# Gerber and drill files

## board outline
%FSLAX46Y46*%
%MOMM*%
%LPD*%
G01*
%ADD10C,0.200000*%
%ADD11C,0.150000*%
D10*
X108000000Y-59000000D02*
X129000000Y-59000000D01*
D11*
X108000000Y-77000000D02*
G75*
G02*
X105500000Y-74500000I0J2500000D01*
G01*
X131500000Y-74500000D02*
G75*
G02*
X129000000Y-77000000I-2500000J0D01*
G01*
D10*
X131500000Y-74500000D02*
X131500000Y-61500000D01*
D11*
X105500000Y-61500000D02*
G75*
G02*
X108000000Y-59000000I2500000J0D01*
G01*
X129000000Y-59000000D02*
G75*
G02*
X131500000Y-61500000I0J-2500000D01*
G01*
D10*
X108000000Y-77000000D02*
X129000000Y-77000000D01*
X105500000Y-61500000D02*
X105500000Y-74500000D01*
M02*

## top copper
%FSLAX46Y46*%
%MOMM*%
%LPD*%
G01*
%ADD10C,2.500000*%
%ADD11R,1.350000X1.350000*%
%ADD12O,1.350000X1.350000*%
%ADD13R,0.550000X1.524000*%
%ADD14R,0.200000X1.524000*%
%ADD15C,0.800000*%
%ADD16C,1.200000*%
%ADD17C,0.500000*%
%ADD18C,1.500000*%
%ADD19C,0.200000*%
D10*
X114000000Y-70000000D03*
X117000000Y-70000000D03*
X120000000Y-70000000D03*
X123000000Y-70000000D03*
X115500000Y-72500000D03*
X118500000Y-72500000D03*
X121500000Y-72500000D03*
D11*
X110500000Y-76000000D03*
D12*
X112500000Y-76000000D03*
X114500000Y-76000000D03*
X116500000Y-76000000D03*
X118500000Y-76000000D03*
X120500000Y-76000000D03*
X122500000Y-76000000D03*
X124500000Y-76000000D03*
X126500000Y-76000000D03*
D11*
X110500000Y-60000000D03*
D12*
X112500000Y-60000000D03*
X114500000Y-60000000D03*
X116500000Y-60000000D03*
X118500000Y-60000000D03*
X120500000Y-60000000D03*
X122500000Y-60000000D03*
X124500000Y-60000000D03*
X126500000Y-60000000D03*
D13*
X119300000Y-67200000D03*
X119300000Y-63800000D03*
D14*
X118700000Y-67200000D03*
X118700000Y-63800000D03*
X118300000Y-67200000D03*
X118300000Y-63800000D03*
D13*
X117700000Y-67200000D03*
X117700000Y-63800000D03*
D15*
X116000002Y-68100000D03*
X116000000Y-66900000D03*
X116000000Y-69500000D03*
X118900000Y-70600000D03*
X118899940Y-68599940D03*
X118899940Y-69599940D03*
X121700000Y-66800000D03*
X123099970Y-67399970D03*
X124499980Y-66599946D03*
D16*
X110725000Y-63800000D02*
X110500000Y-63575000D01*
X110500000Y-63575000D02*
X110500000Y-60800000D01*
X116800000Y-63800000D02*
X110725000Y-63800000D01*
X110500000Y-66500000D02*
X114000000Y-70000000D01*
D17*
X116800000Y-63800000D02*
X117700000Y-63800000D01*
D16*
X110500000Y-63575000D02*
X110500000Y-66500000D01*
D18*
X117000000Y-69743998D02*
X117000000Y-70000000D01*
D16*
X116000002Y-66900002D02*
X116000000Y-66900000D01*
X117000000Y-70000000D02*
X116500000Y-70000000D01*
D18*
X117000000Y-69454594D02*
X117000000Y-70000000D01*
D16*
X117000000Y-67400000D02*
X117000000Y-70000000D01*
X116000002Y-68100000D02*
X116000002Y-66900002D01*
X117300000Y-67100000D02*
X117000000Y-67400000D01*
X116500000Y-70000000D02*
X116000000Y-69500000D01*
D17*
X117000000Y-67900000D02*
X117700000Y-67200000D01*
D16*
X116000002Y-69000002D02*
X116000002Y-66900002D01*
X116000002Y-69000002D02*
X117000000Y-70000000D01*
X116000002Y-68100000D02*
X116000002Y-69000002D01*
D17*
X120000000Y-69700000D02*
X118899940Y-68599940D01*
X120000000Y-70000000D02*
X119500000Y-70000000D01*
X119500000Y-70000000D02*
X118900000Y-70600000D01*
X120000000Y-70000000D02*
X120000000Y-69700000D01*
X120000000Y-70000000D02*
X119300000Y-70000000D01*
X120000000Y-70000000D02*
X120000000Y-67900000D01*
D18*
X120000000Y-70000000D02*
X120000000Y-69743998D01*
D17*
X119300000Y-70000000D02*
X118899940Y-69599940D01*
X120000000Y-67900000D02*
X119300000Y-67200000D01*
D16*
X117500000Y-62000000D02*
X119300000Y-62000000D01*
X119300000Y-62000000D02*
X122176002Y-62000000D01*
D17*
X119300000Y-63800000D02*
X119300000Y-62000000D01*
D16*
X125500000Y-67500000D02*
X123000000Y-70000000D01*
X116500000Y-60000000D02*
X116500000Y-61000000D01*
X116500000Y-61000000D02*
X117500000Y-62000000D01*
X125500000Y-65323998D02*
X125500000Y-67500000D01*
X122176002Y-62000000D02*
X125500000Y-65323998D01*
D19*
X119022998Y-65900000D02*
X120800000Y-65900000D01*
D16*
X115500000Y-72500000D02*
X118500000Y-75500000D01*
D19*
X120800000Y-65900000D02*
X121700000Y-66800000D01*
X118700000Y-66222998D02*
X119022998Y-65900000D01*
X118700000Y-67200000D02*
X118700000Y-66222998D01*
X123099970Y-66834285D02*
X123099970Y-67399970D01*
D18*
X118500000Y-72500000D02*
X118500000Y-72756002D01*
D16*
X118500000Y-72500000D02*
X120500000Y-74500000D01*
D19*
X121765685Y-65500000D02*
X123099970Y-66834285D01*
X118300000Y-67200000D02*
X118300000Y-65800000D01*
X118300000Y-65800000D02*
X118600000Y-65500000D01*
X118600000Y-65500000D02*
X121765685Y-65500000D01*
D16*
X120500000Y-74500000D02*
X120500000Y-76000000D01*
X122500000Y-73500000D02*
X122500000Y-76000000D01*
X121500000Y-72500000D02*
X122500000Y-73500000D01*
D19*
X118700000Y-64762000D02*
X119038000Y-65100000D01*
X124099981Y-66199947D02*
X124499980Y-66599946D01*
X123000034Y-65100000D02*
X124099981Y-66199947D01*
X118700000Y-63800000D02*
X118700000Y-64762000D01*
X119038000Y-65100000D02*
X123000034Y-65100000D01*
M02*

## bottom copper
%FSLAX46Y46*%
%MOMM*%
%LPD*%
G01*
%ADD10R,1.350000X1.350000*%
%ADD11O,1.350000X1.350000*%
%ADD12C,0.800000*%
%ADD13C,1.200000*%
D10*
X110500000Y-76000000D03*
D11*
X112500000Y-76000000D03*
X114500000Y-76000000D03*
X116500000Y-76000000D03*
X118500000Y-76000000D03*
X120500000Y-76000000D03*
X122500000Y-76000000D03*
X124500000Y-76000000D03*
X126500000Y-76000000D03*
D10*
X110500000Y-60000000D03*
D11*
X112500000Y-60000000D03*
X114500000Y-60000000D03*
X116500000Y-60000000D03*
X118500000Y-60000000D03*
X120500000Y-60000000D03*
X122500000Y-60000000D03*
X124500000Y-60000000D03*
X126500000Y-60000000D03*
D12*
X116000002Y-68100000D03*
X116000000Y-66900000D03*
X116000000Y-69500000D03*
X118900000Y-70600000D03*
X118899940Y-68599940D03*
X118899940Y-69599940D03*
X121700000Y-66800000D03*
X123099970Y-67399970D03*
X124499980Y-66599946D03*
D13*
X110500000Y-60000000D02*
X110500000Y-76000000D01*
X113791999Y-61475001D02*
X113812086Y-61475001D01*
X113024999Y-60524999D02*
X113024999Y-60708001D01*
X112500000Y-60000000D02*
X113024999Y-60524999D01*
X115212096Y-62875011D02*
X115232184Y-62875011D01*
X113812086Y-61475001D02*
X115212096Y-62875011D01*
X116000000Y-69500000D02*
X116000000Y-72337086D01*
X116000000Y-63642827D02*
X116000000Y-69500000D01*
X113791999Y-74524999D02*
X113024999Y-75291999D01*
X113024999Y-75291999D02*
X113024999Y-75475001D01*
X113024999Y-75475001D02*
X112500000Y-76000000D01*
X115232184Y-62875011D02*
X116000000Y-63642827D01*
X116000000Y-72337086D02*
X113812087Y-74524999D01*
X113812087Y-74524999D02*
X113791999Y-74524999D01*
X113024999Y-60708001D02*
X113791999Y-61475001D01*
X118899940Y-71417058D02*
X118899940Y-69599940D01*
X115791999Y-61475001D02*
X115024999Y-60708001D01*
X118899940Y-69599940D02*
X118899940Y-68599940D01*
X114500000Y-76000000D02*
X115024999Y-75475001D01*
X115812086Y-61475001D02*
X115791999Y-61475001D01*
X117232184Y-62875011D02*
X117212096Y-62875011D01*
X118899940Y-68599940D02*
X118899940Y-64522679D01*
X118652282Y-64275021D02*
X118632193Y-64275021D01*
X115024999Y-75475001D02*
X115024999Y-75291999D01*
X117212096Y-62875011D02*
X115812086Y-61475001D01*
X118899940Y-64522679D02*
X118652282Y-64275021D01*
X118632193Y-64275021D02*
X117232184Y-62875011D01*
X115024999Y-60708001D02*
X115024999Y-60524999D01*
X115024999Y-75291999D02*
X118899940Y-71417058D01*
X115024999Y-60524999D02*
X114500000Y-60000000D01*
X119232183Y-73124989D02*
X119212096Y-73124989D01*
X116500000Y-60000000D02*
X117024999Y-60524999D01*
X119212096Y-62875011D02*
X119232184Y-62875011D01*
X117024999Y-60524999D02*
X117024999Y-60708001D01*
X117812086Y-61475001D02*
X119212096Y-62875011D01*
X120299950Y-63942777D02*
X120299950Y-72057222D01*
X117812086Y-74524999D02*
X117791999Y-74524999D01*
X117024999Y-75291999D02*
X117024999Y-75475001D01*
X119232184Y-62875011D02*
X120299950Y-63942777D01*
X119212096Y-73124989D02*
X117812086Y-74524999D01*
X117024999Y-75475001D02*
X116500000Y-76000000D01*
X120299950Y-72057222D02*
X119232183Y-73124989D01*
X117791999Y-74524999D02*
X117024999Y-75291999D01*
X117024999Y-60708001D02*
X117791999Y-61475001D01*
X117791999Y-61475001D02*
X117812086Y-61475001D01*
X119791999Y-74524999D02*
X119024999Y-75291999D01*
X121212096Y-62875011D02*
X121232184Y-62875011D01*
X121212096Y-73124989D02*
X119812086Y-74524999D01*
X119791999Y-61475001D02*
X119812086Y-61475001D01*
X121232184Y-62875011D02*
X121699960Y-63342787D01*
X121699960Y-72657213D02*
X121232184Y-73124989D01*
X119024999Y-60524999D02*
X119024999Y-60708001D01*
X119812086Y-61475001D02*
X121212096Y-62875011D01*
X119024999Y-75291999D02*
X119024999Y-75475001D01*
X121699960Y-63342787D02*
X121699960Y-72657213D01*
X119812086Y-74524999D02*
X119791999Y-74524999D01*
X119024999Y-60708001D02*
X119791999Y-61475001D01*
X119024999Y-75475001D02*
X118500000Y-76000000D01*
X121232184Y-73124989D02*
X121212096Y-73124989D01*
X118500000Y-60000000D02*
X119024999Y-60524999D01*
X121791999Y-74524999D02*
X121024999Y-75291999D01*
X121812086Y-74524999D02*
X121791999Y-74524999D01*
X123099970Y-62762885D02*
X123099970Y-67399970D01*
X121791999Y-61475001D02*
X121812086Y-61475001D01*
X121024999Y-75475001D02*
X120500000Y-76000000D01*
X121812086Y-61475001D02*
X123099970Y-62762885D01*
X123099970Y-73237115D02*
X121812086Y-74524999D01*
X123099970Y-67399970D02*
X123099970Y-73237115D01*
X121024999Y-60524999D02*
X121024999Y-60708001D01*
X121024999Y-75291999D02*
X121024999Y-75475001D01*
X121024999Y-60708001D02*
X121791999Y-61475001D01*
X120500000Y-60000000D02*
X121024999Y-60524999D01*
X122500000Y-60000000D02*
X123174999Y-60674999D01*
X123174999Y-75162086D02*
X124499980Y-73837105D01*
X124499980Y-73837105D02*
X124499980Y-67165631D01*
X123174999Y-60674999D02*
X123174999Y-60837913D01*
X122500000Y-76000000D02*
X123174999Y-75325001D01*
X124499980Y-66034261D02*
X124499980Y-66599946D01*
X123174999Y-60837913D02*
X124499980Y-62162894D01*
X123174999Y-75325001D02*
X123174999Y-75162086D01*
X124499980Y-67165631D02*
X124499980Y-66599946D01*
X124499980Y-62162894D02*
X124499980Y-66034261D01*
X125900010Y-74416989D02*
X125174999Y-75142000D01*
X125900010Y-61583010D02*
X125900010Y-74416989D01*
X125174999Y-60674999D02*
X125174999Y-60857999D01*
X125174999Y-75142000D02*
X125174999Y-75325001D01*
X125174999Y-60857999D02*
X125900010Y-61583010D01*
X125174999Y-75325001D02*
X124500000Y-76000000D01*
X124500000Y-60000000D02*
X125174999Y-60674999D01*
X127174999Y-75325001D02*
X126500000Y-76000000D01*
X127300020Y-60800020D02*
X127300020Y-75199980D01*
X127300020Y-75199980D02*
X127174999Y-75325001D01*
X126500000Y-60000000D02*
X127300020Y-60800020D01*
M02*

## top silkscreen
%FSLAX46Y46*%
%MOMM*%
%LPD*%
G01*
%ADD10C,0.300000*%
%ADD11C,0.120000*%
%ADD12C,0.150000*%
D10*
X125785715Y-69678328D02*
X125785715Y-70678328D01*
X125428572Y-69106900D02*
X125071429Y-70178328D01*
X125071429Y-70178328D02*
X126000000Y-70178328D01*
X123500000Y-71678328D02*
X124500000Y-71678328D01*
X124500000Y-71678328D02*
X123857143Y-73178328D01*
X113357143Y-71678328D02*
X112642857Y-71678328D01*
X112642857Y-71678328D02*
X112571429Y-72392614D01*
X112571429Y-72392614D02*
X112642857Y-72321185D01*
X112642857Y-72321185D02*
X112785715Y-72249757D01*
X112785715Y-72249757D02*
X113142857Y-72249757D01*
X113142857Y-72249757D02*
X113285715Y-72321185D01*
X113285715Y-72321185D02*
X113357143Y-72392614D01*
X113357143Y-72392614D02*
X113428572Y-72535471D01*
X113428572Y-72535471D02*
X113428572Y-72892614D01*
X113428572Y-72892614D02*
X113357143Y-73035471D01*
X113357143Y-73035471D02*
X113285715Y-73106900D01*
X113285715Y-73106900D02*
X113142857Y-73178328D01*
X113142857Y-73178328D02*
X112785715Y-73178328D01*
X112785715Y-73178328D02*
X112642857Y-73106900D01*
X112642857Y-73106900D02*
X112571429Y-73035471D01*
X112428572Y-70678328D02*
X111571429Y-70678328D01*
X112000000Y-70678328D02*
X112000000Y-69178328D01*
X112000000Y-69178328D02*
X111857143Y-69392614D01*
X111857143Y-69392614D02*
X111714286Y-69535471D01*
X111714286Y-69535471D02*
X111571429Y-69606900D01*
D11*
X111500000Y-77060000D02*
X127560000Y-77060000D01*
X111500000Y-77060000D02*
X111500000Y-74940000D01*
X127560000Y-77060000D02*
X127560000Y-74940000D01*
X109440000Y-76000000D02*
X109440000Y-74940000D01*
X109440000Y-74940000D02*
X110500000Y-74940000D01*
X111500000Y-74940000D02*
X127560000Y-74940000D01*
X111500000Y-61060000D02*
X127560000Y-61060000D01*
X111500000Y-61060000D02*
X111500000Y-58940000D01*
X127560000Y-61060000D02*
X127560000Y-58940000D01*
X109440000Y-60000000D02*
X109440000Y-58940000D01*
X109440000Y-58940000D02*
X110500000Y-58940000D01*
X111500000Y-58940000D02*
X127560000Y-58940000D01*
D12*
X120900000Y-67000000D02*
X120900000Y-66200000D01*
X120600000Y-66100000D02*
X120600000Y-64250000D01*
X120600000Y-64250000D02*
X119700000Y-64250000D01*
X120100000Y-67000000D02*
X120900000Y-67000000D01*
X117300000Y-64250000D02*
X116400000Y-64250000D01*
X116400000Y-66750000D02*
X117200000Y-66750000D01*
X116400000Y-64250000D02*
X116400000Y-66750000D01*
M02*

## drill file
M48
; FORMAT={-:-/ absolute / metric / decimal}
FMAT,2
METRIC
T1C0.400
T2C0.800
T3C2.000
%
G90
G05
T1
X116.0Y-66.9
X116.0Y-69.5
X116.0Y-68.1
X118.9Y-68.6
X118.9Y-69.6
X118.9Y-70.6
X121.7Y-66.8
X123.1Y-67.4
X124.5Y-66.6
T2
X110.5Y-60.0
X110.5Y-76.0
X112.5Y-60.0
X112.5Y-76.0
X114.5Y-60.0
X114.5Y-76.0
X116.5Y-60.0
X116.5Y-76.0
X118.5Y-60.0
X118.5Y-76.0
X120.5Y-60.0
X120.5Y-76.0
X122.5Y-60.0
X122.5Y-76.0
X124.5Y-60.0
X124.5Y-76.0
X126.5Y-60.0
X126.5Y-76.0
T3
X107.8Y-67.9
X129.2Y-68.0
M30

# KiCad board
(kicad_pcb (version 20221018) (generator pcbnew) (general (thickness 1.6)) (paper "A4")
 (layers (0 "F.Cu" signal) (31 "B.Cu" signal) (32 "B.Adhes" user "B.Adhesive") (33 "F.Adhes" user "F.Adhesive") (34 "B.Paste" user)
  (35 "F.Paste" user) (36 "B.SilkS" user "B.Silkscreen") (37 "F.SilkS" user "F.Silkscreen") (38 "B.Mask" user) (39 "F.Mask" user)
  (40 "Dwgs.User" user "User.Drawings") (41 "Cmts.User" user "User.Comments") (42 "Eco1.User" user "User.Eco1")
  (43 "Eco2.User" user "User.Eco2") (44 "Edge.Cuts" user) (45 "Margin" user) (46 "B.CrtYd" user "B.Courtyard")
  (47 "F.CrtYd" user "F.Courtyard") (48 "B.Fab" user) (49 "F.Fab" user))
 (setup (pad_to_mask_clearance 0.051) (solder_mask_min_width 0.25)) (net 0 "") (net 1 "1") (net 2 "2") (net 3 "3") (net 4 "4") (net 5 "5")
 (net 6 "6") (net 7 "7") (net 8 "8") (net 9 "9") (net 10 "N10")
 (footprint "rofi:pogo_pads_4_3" (layer "F.Cu") (at 118.5 70)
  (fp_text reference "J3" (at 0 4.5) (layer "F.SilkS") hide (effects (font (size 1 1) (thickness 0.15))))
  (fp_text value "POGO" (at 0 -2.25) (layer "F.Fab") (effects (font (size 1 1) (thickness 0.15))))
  (pad "1" smd circle (at -4.5 0) (size 2.5 2.5) (layers "F.Cu" "F.Paste" "F.Mask") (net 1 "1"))
  (pad "2" smd circle (at -1.5 0) (size 2.5 2.5) (layers "F.Cu" "F.Paste" "F.Mask") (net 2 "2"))
  (pad "3" smd circle (at 1.5 0) (size 2.5 2.5) (layers "F.Cu" "F.Paste" "F.Mask") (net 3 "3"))
  (pad "4" smd circle (at 4.5 0) (size 2.5 2.5) (layers "F.Cu" "F.Paste" "F.Mask") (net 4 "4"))
  (pad "5" smd circle (at -3 2.5) (size 2.5 2.5) (layers "F.Cu" "F.Paste" "F.Mask") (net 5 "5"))
  (pad "6" smd circle (at 0 2.5) (size 2.5 2.5) (layers "F.Cu" "F.Paste" "F.Mask") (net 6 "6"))
  (pad "7" smd circle (at 3 2.5) (size 2.5 2.5) (layers "F.Cu" "F.Paste" "F.Mask") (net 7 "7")))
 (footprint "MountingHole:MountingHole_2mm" (layer "F.Cu") (at 129.2 68)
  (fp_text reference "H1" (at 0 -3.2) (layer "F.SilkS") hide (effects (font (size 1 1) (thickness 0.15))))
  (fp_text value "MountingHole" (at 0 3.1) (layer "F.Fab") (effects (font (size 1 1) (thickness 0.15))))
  (pad "" np_thru_hole circle (at 0 0) (size 2 2) (drill 2) (layers "*.Cu" "*.Mask")))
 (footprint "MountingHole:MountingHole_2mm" (layer "F.Cu") (at 107.8 67.9)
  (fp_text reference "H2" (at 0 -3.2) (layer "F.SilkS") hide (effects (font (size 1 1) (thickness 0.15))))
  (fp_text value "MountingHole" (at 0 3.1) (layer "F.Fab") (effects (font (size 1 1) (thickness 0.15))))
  (pad "" np_thru_hole circle (at 0 0) (size 2 2) (drill 2) (layers "*.Cu" "*.Mask")))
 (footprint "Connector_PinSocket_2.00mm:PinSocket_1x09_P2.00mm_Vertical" (layer "F.Cu") (at 110.5 76 90)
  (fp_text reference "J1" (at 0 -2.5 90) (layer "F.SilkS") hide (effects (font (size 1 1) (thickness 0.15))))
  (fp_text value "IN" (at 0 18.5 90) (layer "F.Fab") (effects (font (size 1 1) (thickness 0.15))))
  (fp_line (start -1.06 1) (end -1.06 17.06) (stroke (width 0.12) (type solid)) (layer "F.SilkS"))
  (fp_line (start -1.06 1) (end 1.06 1) (stroke (width 0.12) (type solid)) (layer "F.SilkS"))
  (fp_line (start -1.06 17.06) (end 1.06 17.06) (stroke (width 0.12) (type solid)) (layer "F.SilkS"))
  (fp_line (start 0 -1.06) (end 1.06 -1.06) (stroke (width 0.12) (type solid)) (layer "F.SilkS"))
  (fp_line (start 1.06 -1.06) (end 1.06 0) (stroke (width 0.12) (type solid)) (layer "F.SilkS"))
  (fp_line (start 1.06 1) (end 1.06 17.06) (stroke (width 0.12) (type solid)) (layer "F.SilkS"))
  (pad "1" thru_hole rect (at 0 0 90) (size 1.35 1.35) (drill 0.8) (layers "*.Cu" "*.Mask") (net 1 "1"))
  (pad "2" thru_hole oval (at 0 2 90) (size 1.35 1.35) (drill 0.8) (layers "*.Cu" "*.Mask") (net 2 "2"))
  (pad "3" thru_hole oval (at 0 4 90) (size 1.35 1.35) (drill 0.8) (layers "*.Cu" "*.Mask") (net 3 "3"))
  (pad "4" thru_hole oval (at 0 6 90) (size 1.35 1.35) (drill 0.8) (layers "*.Cu" "*.Mask") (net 4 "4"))
  (pad "5" thru_hole oval (at 0 8 90) (size 1.35 1.35) (drill 0.8) (layers "*.Cu" "*.Mask") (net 5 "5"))
  (pad "6" thru_hole oval (at 0 10 90) (size 1.35 1.35) (drill 0.8) (layers "*.Cu" "*.Mask") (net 6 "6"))
  (pad "7" thru_hole oval (at 0 12 90) (size 1.35 1.35) (drill 0.8) (layers "*.Cu" "*.Mask") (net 7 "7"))
  (pad "8" thru_hole oval (at 0 14 90) (size 1.35 1.35) (drill 0.8) (layers "*.Cu" "*.Mask") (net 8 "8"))
  (pad "9" thru_hole oval (at 0 16 90) (size 1.35 1.35) (drill 0.8) (layers "*.Cu" "*.Mask") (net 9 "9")))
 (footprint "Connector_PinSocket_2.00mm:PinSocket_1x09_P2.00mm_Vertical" (layer "F.Cu") (at 110.5 60 90)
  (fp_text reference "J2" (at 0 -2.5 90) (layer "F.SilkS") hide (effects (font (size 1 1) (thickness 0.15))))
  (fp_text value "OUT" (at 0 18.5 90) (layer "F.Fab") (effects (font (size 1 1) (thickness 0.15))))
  (fp_line (start -1.06 1) (end -1.06 17.06) (stroke (width 0.12) (type solid)) (layer "F.SilkS"))
  (fp_line (start -1.06 1) (end 1.06 1) (stroke (width 0.12) (type solid)) (layer "F.SilkS"))
  (fp_line (start -1.06 17.06) (end 1.06 17.06) (stroke (width 0.12) (type solid)) (layer "F.SilkS"))
  (fp_line (start 0 -1.06) (end 1.06 -1.06) (stroke (width 0.12) (type solid)) (layer "F.SilkS"))
  (fp_line (start 1.06 -1.06) (end 1.06 0) (stroke (width 0.12) (type solid)) (layer "F.SilkS"))
  (fp_line (start 1.06 1) (end 1.06 17.06) (stroke (width 0.12) (type solid)) (layer "F.SilkS"))
  (pad "1" thru_hole rect (at 0 0 90) (size 1.35 1.35) (drill 0.8) (layers "*.Cu" "*.Mask") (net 1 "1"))
  (pad "2" thru_hole oval (at 0 2 90) (size 1.35 1.35) (drill 0.8) (layers "*.Cu" "*.Mask") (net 2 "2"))
  (pad "3" thru_hole oval (at 0 4 90) (size 1.35 1.35) (drill 0.8) (layers "*.Cu" "*.Mask") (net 3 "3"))
  (pad "4" thru_hole oval (at 0 6 90) (size 1.35 1.35) (drill 0.8) (layers "*.Cu" "*.Mask") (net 4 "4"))
  (pad "5" thru_hole oval (at 0 8 90) (size 1.35 1.35) (drill 0.8) (layers "*.Cu" "*.Mask") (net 5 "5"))
  (pad "6" thru_hole oval (at 0 10 90) (size 1.35 1.35) (drill 0.8) (layers "*.Cu" "*.Mask") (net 6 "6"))
  (pad "7" thru_hole oval (at 0 12 90) (size 1.35 1.35) (drill 0.8) (layers "*.Cu" "*.Mask") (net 7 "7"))
  (pad "8" thru_hole oval (at 0 14 90) (size 1.35 1.35) (drill 0.8) (layers "*.Cu" "*.Mask") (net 8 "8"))
  (pad "9" thru_hole oval (at 0 16 90) (size 1.35 1.35) (drill 0.8) (layers "*.Cu" "*.Mask") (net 9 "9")))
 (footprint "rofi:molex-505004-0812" (layer "F.Cu") (at 118.5 65.5 180)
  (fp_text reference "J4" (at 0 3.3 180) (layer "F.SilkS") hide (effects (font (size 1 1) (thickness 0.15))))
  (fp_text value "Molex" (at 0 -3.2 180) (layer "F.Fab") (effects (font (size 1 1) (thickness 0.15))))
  (fp_line (start -2.4 -1.5) (end -2.4 -0.7) (stroke (width 0.15) (type solid)) (layer "F.SilkS"))
  (fp_line (start -2.1 -0.6) (end -2.1 1.25) (stroke (width 0.15) (type solid)) (layer "F.SilkS"))
  (fp_line (start -2.1 1.25) (end -1.2 1.25) (stroke (width 0.15) (type solid)) (layer "F.SilkS"))
  (fp_line (start -1.6 -1.5) (end -2.4 -1.5) (stroke (width 0.15) (type solid)) (layer "F.SilkS"))
  (fp_line (start 1.2 1.25) (end 2.1 1.25) (stroke (width 0.15) (type solid)) (layer "F.SilkS"))
  (fp_line (start 2.1 -1.25) (end 1.3 -1.25) (stroke (width 0.15) (type solid)) (layer "F.SilkS"))
  (fp_line (start 2.1 1.25) (end 2.1 -1.25) (stroke (width 0.15) (type solid)) (layer "F.SilkS"))
  (pad "1" smd rect (at -0.8 -1.7 180) (size 0.55 1.524) (layers "F.Cu" "F.Paste" "F.Mask") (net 3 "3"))
  (pad "2" smd rect (at -0.8 1.7 180) (size 0.55 1.524) (layers "F.Cu" "F.Paste" "F.Mask") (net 4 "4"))
  (pad "3" smd rect (at -0.2 -1.7 180) (size 0.2 1.524) (layers "F.Cu" "F.Paste" "F.Mask") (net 5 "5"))
  (pad "4" smd rect (at -0.2 1.7 180) (size 0.2 1.524) (layers "F.Cu" "F.Paste" "F.Mask") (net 7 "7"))
  (pad "5" smd rect (at 0.2 -1.7 180) (size 0.2 1.524) (layers "F.Cu" "F.Paste" "F.Mask") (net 6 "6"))
  (pad "6" smd rect (at 0.2 1.7 180) (size 0.2 1.524) (layers "F.Cu" "F.Paste" "F.Mask") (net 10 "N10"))
  (pad "7" smd rect (at 0.8 -1.7 180) (size 0.55 1.524) (layers "F.Cu" "F.Paste" "F.Mask") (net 2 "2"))
  (pad "8" smd rect (at 0.8 1.7 180) (size 0.55 1.524) (layers "F.Cu" "F.Paste" "F.Mask") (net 1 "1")))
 (gr_line (start 108 59) (end 129 59) (stroke (width 0.2) (type solid)) (layer "Edge.Cuts"))
 (gr_arc (start 108 77) (mid 106.232233 76.267767) (end 105.5 74.5) (stroke (width 0.15) (type solid)) (layer "Edge.Cuts"))
 (gr_arc (start 131.5 74.5) (mid 130.767767 76.267767) (end 129 77) (stroke (width 0.15) (type solid)) (layer "Edge.Cuts"))
 (gr_line (start 131.5 74.5) (end 131.5 61.5) (stroke (width 0.2) (type solid)) (layer "Edge.Cuts"))
 (gr_arc (start 105.5 61.5) (mid 106.232233 59.732233) (end 108 59) (stroke (width 0.15) (type solid)) (layer "Edge.Cuts"))
 (gr_arc (start 129 59) (mid 130.767767 59.732233) (end 131.5 61.5) (stroke (width 0.15) (type solid)) (layer "Edge.Cuts"))
 (gr_line (start 108 77) (end 129 77) (stroke (width 0.2) (type solid)) (layer "Edge.Cuts"))
 (gr_line (start 105.5 61.5) (end 105.5 74.5) (stroke (width 0.2) (type solid)) (layer "Edge.Cuts"))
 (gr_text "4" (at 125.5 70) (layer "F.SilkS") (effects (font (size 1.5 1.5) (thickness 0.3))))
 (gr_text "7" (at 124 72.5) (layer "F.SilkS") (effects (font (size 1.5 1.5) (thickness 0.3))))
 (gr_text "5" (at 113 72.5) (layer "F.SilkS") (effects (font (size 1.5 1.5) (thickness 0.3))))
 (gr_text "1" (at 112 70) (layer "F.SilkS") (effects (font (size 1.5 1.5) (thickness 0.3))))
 (segment (start 110.725 63.8) (end 110.5 63.575) (width 1.2) (layer "F.Cu") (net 1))
 (segment (start 110.5 63.575) (end 110.5 60.8) (width 1.2) (layer "F.Cu") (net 1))
 (segment (start 116.8 63.8) (end 110.725 63.8) (width 1.2) (layer "F.Cu") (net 1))
 (segment (start 110.5 66.5) (end 114 70) (width 1.2) (layer "F.Cu") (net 1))
 (segment (start 116.8 63.8) (end 117.7 63.8) (width 0.5) (layer "F.Cu") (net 1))
 (segment (start 110.5 63.575) (end 110.5 66.5) (width 1.2) (layer "F.Cu") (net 1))
 (segment (start 110.5 60) (end 110.5 76) (width 1.2) (layer "B.Cu") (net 1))
 (segment (start 117 69.743998) (end 117 70) (width 1.5) (layer "F.Cu") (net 2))
 (segment (start 116.000002 66.900002) (end 116 66.9) (width 1.2) (layer "F.Cu") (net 2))
 (segment (start 117 70) (end 116.5 70) (width 1.2) (layer "F.Cu") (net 2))
 (segment (start 117 69.454594) (end 117 70) (width 1.5) (layer "F.Cu") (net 2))
 (segment (start 117 67.4) (end 117 70) (width 1.2) (layer "F.Cu") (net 2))
 (segment (start 116.000002 68.1) (end 116.000002 66.900002) (width 1.2) (layer "F.Cu") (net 2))
 (segment (start 117.3 67.1) (end 117 67.4) (width 1.2) (layer "F.Cu") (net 2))
 (segment (start 116.5 70) (end 116 69.5) (width 1.2) (layer "F.Cu") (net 2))
 (segment (start 117 67.9) (end 117.7 67.2) (width 0.5) (layer "F.Cu") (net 2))
 (segment (start 116.000002 69.000002) (end 116.000002 66.900002) (width 1.2) (layer "F.Cu") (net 2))
 (segment (start 116.000002 69.000002) (end 117 70) (width 1.2) (layer "F.Cu") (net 2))
 (segment (start 116.000002 68.1) (end 116.000002 69.000002) (width 1.2) (layer "F.Cu") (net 2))
 (via (at 116.000002 68.1) (size 0.8) (drill 0.4) (layers "F.Cu" "B.Cu") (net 2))
 (via (at 116 66.9) (size 0.8) (drill 0.4) (layers "F.Cu" "B.Cu") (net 2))
 (via (at 116 69.5) (size 0.8) (drill 0.4) (layers "F.Cu" "B.Cu") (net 2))
 (segment (start 113.791999 61.475001) (end 113.812086 61.475001) (width 1.2) (layer "B.Cu") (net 2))
 (segment (start 113.024999 60.524999) (end 113.024999 60.708001) (width 1.2) (layer "B.Cu") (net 2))
 (segment (start 112.5 60) (end 113.024999 60.524999) (width 1.2) (layer "B.Cu") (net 2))
 (segment (start 115.212096 62.875011) (end 115.232184 62.875011) (width 1.2) (layer "B.Cu") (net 2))
 (segment (start 113.812086 61.475001) (end 115.212096 62.875011) (width 1.2) (layer "B.Cu") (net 2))
 (segment (start 116 69.5) (end 116 72.337086) (width 1.2) (layer "B.Cu") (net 2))
 (segment (start 116 63.642827) (end 116 69.5) (width 1.2) (layer "B.Cu") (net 2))
 (segment (start 113.791999 74.524999) (end 113.024999 75.291999) (width 1.2) (layer "B.Cu") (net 2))
 (segment (start 113.024999 75.291999) (end 113.024999 75.475001) (width 1.2) (layer "B.Cu") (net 2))
 (segment (start 113.024999 75.475001) (end 112.5 76) (width 1.2) (layer "B.Cu") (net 2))
 (segment (start 115.232184 62.875011) (end 116 63.642827) (width 1.2) (layer "B.Cu") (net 2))
 (segment (start 116 72.337086) (end 113.812087 74.524999) (width 1.2) (layer "B.Cu") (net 2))
 (segment (start 113.812087 74.524999) (end 113.791999 74.524999) (width 1.2) (layer "B.Cu") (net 2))
 (segment (start 113.024999 60.708001) (end 113.791999 61.475001) (width 1.2) (layer "B.Cu") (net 2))
 (segment (start 120 69.7) (end 118.89994 68.59994) (width 0.5) (layer "F.Cu") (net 3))
 (segment (start 120 70) (end 119.5 70) (width 0.5) (layer "F.Cu") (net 3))
 (segment (start 119.5 70) (end 118.9 70.6) (width 0.5) (layer "F.Cu") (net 3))
 (segment (start 120 70) (end 120 69.7) (width 0.5) (layer "F.Cu") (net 3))
 (segment (start 120 70) (end 119.3 70) (width 0.5) (layer "F.Cu") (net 3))
 (segment (start 120 70) (end 120 67.9) (width 0.5) (layer "F.Cu") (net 3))
 (segment (start 120 70) (end 120 69.743998) (width 1.5) (layer "F.Cu") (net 3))
 (segment (start 119.3 70) (end 118.89994 69.59994) (width 0.5) (layer "F.Cu") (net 3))
 (segment (start 120 67.9) (end 119.3 67.2) (width 0.5) (layer "F.Cu") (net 3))
 (via (at 118.9 70.6) (size 0.8) (drill 0.4) (layers "F.Cu" "B.Cu") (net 3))
 (via (at 118.89994 68.59994) (size 0.8) (drill 0.4) (layers "F.Cu" "B.Cu") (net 3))
 (via (at 118.89994 69.59994) (size 0.8) (drill 0.4) (layers "F.Cu" "B.Cu") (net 3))
 (segment (start 118.89994 71.417058) (end 118.89994 69.59994) (width 1.2) (layer "B.Cu") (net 3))
 (segment (start 115.791999 61.475001) (end 115.024999 60.708001) (width 1.2) (layer "B.Cu") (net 3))
 (segment (start 118.89994 69.59994) (end 118.89994 68.59994) (width 1.2) (layer "B.Cu") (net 3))
 (segment (start 114.5 76) (end 115.024999 75.475001) (width 1.2) (layer "B.Cu") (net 3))
 (segment (start 115.812086 61.475001) (end 115.791999 61.475001) (width 1.2) (layer "B.Cu") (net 3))
 (segment (start 117.232184 62.875011) (end 117.212096 62.875011) (width 1.2) (layer "B.Cu") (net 3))
 (segment (start 118.89994 68.59994) (end 118.89994 64.522679) (width 1.2) (layer "B.Cu") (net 3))
 (segment (start 118.652282 64.275021) (end 118.632193 64.275021) (width 1.2) (layer "B.Cu") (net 3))
 (segment (start 115.024999 75.475001) (end 115.024999 75.291999) (width 1.2) (layer "B.Cu") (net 3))
 (segment (start 117.212096 62.875011) (end 115.812086 61.475001) (width 1.2) (layer "B.Cu") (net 3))
 (segment (start 118.89994 64.522679) (end 118.652282 64.275021) (width 1.2) (layer "B.Cu") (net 3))
 (segment (start 118.632193 64.275021) (end 117.232184 62.875011) (width 1.2) (layer "B.Cu") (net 3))
 (segment (start 115.024999 60.708001) (end 115.024999 60.524999) (width 1.2) (layer "B.Cu") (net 3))
 (segment (start 115.024999 75.291999) (end 118.89994 71.417058) (width 1.2) (layer "B.Cu") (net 3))
 (segment (start 115.024999 60.524999) (end 114.5 60) (width 1.2) (layer "B.Cu") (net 3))
 (segment (start 117.5 62) (end 119.3 62) (width 1.2) (layer "F.Cu") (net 4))
 (segment (start 119.3 62) (end 122.176002 62) (width 1.2) (layer "F.Cu") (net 4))
 (segment (start 119.3 63.8) (end 119.3 62) (width 0.5) (layer "F.Cu") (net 4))
 (segment (start 125.5 67.5) (end 123 70) (width 1.2) (layer "F.Cu") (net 4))
 (segment (start 116.5 60) (end 116.5 61) (width 1.2) (layer "F.Cu") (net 4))
 (segment (start 116.5 61) (end 117.5 62) (width 1.2) (layer "F.Cu") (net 4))
 (segment (start 125.5 65.323998) (end 125.5 67.5) (width 1.2) (layer "F.Cu") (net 4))
 (segment (start 122.176002 62) (end 125.5 65.323998) (width 1.2) (layer "F.Cu") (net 4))
 (segment (start 119.232183 73.124989) (end 119.212096 73.124989) (width 1.2) (layer "B.Cu") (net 4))
 (segment (start 116.5 60) (end 117.024999 60.524999) (width 1.2) (layer "B.Cu") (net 4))
 (segment (start 119.212096 62.875011) (end 119.232184 62.875011) (width 1.2) (layer "B.Cu") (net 4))
 (segment (start 117.024999 60.524999) (end 117.024999 60.708001) (width 1.2) (layer "B.Cu") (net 4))
 (segment (start 117.812086 61.475001) (end 119.212096 62.875011) (width 1.2) (layer "B.Cu") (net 4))
 (segment (start 120.29995 63.942777) (end 120.29995 72.057222) (width 1.2) (layer "B.Cu") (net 4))
 (segment (start 117.812086 74.524999) (end 117.791999 74.524999) (width 1.2) (layer "B.Cu") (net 4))
 (segment (start 117.024999 75.291999) (end 117.024999 75.475001) (width 1.2) (layer "B.Cu") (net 4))
 (segment (start 119.232184 62.875011) (end 120.29995 63.942777) (width 1.2) (layer "B.Cu") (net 4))
 (segment (start 119.212096 73.124989) (end 117.812086 74.524999) (width 1.2) (layer "B.Cu") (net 4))
 (segment (start 117.024999 75.475001) (end 116.5 76) (width 1.2) (layer "B.Cu") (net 4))
 (segment (start 120.29995 72.057222) (end 119.232183 73.124989) (width 1.2) (layer "B.Cu") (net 4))
 (segment (start 117.791999 74.524999) (end 117.024999 75.291999) (width 1.2) (layer "B.Cu") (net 4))
 (segment (start 117.024999 60.708001) (end 117.791999 61.475001) (width 1.2) (layer "B.Cu") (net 4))
 (segment (start 117.791999 61.475001) (end 117.812086 61.475001) (width 1.2) (layer "B.Cu") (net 4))
 (segment (start 119.022998 65.9) (end 120.8 65.9) (width 0.2) (layer "F.Cu") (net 5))
 (segment (start 115.5 72.5) (end 118.5 75.5) (width 1.2) (layer "F.Cu") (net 5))
 (segment (start 120.8 65.9) (end 121.7 66.8) (width 0.2) (layer "F.Cu") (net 5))
 (segment (start 118.7 66.222998) (end 119.022998 65.9) (width 0.2) (layer "F.Cu") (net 5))
 (segment (start 118.7 67.2) (end 118.7 66.222998) (width 0.2) (layer "F.Cu") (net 5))
 (via (at 121.7 66.8) (size 0.8) (drill 0.4) (layers "F.Cu" "B.Cu") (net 5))
 (segment (start 119.791999 74.524999) (end 119.024999 75.291999) (width 1.2) (layer "B.Cu") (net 5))
 (segment (start 121.212096 62.875011) (end 121.232184 62.875011) (width 1.2) (layer "B.Cu") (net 5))
 (segment (start 121.212096 73.124989) (end 119.812086 74.524999) (width 1.2) (layer "B.Cu") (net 5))
 (segment (start 119.791999 61.475001) (end 119.812086 61.475001) (width 1.2) (layer "B.Cu") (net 5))
 (segment (start 121.232184 62.875011) (end 121.69996 63.342787) (width 1.2) (layer "B.Cu") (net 5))
 (segment (start 121.69996 72.657213) (end 121.232184 73.124989) (width 1.2) (layer "B.Cu") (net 5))
 (segment (start 119.024999 60.524999) (end 119.024999 60.708001) (width 1.2) (layer "B.Cu") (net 5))
 (segment (start 119.812086 61.475001) (end 121.212096 62.875011) (width 1.2) (layer "B.Cu") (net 5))
 (segment (start 119.024999 75.291999) (end 119.024999 75.475001) (width 1.2) (layer "B.Cu") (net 5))
 (segment (start 121.69996 63.342787) (end 121.69996 72.657213) (width 1.2) (layer "B.Cu") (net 5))
 (segment (start 119.812086 74.524999) (end 119.791999 74.524999) (width 1.2) (layer "B.Cu") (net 5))
 (segment (start 119.024999 60.708001) (end 119.791999 61.475001) (width 1.2) (layer "B.Cu") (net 5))
 (segment (start 119.024999 75.475001) (end 118.5 76) (width 1.2) (layer "B.Cu") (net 5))
 (segment (start 121.232184 73.124989) (end 121.212096 73.124989) (width 1.2) (layer "B.Cu") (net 5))
 (segment (start 118.5 60) (end 119.024999 60.524999) (width 1.2) (layer "B.Cu") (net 5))
 (segment (start 123.09997 66.834285) (end 123.09997 67.39997) (width 0.2) (layer "F.Cu") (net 6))
 (segment (start 118.5 72.5) (end 118.5 72.756002) (width 1.5) (layer "F.Cu") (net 6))
 (segment (start 118.5 72.5) (end 120.5 74.5) (width 1.2) (layer "F.Cu") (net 6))
 (segment (start 121.765685 65.5) (end 123.09997 66.834285) (width 0.2) (layer "F.Cu") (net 6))
 (segment (start 118.3 67.2) (end 118.3 65.8) (width 0.2) (layer "F.Cu") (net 6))
 (segment (start 118.3 65.8) (end 118.6 65.5) (width 0.2) (layer "F.Cu") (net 6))
 (segment (start 118.6 65.5) (end 121.765685 65.5) (width 0.2) (layer "F.Cu") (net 6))
 (segment (start 120.5 74.5) (end 120.5 76) (width 1.2) (layer "F.Cu") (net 6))
 (via (at 123.09997 67.39997) (size 0.8) (drill 0.4) (layers "F.Cu" "B.Cu") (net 6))
 (segment (start 121.791999 74.524999) (end 121.024999 75.291999) (width 1.2) (layer "B.Cu") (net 6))
 (segment (start 121.812086 74.524999) (end 121.791999 74.524999) (width 1.2) (layer "B.Cu") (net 6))
 (segment (start 123.09997 62.762885) (end 123.09997 67.39997) (width 1.2) (layer "B.Cu") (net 6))
 (segment (start 121.791999 61.475001) (end 121.812086 61.475001) (width 1.2) (layer "B.Cu") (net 6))
 (segment (start 121.024999 75.475001) (end 120.5 76) (width 1.2) (layer "B.Cu") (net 6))
 (segment (start 121.812086 61.475001) (end 123.09997 62.762885) (width 1.2) (layer "B.Cu") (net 6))
 (segment (start 123.09997 73.237115) (end 121.812086 74.524999) (width 1.2) (layer "B.Cu") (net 6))
 (segment (start 123.09997 67.39997) (end 123.09997 73.237115) (width 1.2) (layer "B.Cu") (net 6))
 (segment (start 121.024999 60.524999) (end 121.024999 60.708001) (width 1.2) (layer "B.Cu") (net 6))
 (segment (start 121.024999 75.291999) (end 121.024999 75.475001) (width 1.2) (layer "B.Cu") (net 6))
 (segment (start 121.024999 60.708001) (end 121.791999 61.475001) (width 1.2) (layer "B.Cu") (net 6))
 (segment (start 120.5 60) (end 121.024999 60.524999) (width 1.2) (layer "B.Cu") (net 6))
 (segment (start 122.5 73.5) (end 122.5 76) (width 1.2) (layer "F.Cu") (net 7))
 (segment (start 121.5 72.5) (end 122.5 73.5) (width 1.2) (layer "F.Cu") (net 7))
 (segment (start 118.7 64.762) (end 119.038 65.1) (width 0.2) (layer "F.Cu") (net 7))
 (segment (start 124.099981 66.199947) (end 124.49998 66.599946) (width 0.2) (layer "F.Cu") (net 7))
 (segment (start 123.000034 65.1) (end 124.099981 66.199947) (width 0.2) (layer "F.Cu") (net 7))
 (segment (start 118.7 63.8) (end 118.7 64.762) (width 0.2) (layer "F.Cu") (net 7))
 (segment (start 119.038 65.1) (end 123.000034 65.1) (width 0.2) (layer "F.Cu") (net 7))
 (via (at 124.49998 66.599946) (size 0.8) (drill 0.4) (layers "F.Cu" "B.Cu") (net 7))
 (segment (start 122.5 60) (end 123.174999 60.674999) (width 1.2) (layer "B.Cu") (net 7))
 (segment (start 123.174999 75.162086) (end 124.49998 73.837105) (width 1.2) (layer "B.Cu") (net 7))
 (segment (start 124.49998 73.837105) (end 124.49998 67.165631) (width 1.2) (layer "B.Cu") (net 7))
 (segment (start 123.174999 60.674999) (end 123.174999 60.837913) (width 1.2) (layer "B.Cu") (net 7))
 (segment (start 122.5 76) (end 123.174999 75.325001) (width 1.2) (layer "B.Cu") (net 7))
 (segment (start 124.49998 66.034261) (end 124.49998 66.599946) (width 1.2) (layer "B.Cu") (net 7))
 (segment (start 123.174999 60.837913) (end 124.49998 62.162894) (width 1.2) (layer "B.Cu") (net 7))
 (segment (start 123.174999 75.325001) (end 123.174999 75.162086) (width 1.2) (layer "B.Cu") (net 7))
 (segment (start 124.49998 67.165631) (end 124.49998 66.599946) (width 1.2) (layer "B.Cu") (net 7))
 (segment (start 124.49998 62.162894) (end 124.49998 66.034261) (width 1.2) (layer "B.Cu") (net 7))
 (segment (start 125.90001 74.416989) (end 125.174999 75.142) (width 1.2) (layer "B.Cu") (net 8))
 (segment (start 125.90001 61.58301) (end 125.90001 74.416989) (width 1.2) (layer "B.Cu") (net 8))
 (segment (start 125.174999 60.674999) (end 125.174999 60.857999) (width 1.2) (layer "B.Cu") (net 8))
 (segment (start 125.174999 75.142) (end 125.174999 75.325001) (width 1.2) (layer "B.Cu") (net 8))
 (segment (start 125.174999 60.857999) (end 125.90001 61.58301) (width 1.2) (layer "B.Cu") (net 8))
 (segment (start 125.174999 75.325001) (end 124.5 76) (width 1.2) (layer "B.Cu") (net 8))
 (segment (start 124.5 60) (end 125.174999 60.674999) (width 1.2) (layer "B.Cu") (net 8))
 (segment (start 127.174999 75.325001) (end 126.5 76) (width 1.2) (layer "B.Cu") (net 9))
 (segment (start 127.30002 60.80002) (end 127.30002 75.19998) (width 1.2) (layer "B.Cu") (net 9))
 (segment (start 127.30002 75.19998) (end 127.174999 75.325001) (width 1.2) (layer "B.Cu") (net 9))
 (segment (start 126.5 60) (end 127.30002 60.80002) (width 1.2) (layer "B.Cu") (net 9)))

